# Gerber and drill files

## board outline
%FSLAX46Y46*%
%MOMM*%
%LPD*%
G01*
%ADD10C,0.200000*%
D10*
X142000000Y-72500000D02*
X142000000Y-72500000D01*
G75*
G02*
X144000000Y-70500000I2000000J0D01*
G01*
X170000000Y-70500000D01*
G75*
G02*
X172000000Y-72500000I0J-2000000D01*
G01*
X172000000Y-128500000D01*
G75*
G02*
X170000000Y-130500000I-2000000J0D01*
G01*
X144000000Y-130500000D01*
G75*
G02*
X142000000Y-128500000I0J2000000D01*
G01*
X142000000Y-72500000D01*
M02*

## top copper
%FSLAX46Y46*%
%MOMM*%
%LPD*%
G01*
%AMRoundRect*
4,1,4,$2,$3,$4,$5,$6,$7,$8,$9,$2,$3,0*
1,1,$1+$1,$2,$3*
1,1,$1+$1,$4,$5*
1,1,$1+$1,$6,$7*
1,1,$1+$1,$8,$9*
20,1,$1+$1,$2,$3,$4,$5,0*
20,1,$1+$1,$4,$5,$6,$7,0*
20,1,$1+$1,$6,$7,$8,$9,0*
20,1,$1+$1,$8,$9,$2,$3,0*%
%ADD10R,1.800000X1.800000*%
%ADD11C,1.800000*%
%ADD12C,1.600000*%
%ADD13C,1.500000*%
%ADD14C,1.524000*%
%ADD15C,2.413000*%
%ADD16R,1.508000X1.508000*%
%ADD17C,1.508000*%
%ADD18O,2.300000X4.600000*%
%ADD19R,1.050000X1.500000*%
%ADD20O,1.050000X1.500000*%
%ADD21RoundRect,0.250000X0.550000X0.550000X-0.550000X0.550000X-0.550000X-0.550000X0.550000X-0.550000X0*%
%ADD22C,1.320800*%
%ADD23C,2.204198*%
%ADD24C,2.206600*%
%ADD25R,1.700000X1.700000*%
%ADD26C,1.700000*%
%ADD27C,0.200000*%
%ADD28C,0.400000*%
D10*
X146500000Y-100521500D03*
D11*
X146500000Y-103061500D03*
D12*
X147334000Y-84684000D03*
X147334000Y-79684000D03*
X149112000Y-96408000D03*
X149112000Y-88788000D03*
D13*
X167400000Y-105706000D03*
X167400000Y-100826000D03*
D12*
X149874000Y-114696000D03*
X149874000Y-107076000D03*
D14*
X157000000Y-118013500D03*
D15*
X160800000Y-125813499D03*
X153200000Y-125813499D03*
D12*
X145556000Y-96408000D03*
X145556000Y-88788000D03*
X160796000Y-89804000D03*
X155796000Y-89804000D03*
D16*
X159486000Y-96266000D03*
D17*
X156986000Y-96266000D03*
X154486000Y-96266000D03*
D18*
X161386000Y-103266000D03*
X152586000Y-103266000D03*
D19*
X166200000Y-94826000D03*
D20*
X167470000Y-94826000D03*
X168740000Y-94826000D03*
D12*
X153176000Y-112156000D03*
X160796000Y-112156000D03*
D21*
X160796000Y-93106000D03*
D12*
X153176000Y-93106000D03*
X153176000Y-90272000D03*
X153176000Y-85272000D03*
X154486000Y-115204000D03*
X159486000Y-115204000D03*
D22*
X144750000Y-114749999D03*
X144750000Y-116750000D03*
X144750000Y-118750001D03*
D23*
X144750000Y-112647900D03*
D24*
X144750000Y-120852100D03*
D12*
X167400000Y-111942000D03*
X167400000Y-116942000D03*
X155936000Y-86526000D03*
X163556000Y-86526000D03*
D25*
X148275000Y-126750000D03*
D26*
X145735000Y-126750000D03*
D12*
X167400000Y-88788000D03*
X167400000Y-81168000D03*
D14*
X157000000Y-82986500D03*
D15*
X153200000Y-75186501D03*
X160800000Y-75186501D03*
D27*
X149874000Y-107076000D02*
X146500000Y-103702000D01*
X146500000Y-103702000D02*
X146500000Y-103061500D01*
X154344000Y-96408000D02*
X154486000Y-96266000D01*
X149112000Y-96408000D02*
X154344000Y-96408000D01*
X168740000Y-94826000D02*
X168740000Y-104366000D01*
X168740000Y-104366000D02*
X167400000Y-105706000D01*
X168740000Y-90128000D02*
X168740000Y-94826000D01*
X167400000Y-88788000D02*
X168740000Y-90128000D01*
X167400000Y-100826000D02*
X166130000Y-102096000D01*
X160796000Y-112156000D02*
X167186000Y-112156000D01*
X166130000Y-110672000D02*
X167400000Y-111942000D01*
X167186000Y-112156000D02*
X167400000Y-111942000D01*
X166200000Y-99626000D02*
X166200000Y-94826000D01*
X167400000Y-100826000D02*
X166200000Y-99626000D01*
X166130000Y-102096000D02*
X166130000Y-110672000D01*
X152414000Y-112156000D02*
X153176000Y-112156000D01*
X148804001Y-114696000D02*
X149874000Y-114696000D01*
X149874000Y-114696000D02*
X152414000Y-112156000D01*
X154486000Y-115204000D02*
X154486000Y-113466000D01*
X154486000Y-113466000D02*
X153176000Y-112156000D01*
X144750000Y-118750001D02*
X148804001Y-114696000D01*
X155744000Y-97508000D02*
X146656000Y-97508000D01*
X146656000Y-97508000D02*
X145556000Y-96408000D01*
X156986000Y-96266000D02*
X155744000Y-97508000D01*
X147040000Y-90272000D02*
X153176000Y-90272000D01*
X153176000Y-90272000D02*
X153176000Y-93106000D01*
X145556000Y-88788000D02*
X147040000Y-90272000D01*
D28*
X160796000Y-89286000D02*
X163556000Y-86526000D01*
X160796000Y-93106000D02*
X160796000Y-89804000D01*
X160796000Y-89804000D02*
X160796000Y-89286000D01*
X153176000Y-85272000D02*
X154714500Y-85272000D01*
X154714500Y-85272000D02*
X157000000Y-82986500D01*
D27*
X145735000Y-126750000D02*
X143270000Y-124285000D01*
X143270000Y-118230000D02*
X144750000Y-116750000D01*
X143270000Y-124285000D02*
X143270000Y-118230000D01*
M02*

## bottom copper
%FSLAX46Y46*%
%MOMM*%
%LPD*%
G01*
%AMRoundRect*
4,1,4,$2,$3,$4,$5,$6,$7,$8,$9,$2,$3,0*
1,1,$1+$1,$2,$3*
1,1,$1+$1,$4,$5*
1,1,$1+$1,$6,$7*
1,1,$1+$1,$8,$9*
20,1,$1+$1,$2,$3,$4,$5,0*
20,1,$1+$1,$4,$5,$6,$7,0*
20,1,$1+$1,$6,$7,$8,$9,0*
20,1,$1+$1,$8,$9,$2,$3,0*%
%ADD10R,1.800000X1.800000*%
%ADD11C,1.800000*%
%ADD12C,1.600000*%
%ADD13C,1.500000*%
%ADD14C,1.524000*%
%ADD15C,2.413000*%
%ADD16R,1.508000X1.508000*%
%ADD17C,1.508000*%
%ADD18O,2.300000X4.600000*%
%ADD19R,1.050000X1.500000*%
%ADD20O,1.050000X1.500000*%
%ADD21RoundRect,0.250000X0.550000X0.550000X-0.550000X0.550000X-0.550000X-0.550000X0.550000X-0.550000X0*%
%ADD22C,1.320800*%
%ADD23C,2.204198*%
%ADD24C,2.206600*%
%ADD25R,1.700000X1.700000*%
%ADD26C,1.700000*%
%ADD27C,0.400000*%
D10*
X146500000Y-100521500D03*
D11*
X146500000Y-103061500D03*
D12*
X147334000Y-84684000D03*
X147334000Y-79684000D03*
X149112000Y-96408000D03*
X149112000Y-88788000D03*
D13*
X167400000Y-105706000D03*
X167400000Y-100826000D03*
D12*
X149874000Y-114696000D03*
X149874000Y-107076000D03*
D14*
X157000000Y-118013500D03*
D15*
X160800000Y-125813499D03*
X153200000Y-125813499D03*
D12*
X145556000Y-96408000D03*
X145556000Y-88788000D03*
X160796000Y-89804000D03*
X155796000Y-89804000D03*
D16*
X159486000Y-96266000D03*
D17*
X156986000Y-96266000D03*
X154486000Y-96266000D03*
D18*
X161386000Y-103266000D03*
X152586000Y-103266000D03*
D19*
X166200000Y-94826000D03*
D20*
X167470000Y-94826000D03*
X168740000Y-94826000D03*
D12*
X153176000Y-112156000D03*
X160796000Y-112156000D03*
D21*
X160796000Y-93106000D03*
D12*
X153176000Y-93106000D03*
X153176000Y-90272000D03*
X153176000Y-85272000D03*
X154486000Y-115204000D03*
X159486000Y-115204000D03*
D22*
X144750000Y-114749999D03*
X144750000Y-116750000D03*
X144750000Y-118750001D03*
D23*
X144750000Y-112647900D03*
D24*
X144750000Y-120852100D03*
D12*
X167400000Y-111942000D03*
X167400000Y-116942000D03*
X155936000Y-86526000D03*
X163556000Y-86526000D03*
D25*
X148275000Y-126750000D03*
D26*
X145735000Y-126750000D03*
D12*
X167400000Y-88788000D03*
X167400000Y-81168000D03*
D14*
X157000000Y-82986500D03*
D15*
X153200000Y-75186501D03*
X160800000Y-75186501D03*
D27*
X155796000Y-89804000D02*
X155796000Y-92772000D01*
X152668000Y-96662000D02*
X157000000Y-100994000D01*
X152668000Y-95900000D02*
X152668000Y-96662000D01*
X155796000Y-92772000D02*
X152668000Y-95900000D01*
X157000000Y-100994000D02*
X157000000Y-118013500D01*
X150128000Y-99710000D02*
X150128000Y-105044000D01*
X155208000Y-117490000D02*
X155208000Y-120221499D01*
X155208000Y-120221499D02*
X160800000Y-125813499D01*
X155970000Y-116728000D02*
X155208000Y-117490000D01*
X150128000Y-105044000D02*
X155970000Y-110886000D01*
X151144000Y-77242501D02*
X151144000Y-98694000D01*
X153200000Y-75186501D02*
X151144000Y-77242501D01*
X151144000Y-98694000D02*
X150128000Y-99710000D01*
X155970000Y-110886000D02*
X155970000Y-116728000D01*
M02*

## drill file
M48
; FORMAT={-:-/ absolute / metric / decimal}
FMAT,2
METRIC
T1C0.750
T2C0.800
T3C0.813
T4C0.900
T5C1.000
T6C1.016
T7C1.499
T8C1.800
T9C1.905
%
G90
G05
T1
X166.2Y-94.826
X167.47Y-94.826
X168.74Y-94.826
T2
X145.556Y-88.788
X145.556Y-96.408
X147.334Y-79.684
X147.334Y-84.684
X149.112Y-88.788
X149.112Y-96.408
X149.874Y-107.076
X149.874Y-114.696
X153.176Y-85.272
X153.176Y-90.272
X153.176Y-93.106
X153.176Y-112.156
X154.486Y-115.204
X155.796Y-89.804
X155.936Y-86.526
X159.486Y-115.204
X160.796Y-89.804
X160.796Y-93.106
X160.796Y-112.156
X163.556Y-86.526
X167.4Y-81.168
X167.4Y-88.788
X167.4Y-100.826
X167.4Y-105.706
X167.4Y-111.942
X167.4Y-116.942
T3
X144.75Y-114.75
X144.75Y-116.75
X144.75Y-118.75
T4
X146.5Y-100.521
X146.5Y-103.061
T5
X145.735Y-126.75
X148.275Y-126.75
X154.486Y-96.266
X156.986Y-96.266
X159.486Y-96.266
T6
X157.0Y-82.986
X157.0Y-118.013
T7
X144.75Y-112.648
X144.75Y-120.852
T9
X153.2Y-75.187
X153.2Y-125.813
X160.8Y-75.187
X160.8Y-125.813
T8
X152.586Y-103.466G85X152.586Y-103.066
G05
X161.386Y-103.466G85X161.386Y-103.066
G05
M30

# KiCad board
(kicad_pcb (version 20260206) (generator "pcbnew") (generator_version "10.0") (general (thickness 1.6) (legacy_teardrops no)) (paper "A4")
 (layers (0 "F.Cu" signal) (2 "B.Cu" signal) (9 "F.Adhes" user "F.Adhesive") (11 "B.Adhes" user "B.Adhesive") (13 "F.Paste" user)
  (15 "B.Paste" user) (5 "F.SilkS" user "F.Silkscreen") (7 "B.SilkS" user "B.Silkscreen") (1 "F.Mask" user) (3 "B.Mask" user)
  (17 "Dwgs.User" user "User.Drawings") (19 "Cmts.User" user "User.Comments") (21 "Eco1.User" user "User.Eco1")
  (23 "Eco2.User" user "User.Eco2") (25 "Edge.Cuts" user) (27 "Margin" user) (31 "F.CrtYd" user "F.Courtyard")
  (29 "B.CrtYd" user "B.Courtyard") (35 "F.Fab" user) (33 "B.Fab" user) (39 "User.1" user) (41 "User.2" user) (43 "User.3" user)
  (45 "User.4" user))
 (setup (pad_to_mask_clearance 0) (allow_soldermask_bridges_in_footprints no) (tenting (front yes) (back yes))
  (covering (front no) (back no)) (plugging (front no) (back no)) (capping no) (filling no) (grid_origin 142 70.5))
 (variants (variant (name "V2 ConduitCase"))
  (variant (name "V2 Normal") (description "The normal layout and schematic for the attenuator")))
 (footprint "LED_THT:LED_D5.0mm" (layer "F.Cu") (at 146.5 100.5215 -90)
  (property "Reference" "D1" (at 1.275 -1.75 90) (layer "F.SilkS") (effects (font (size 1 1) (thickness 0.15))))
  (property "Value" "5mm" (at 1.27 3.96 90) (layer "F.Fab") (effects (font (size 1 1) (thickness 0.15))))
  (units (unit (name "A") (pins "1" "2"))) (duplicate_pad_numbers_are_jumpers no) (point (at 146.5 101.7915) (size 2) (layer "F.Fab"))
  (pad "1" thru_hole rect (at 0 0 270) (size 1.8 1.8) (drill 0.9) (layers "*.Cu" "*.Mask") (remove_unused_layers no) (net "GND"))
  (pad "2" thru_hole circle (at 2.54 0 270) (size 1.8 1.8) (drill 0.9) (layers "*.Cu" "*.Mask") (remove_unused_layers no) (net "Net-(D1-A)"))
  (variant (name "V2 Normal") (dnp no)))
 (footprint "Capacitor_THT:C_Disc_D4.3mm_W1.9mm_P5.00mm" (layer "F.Cu") (at 147.334 84.684 90)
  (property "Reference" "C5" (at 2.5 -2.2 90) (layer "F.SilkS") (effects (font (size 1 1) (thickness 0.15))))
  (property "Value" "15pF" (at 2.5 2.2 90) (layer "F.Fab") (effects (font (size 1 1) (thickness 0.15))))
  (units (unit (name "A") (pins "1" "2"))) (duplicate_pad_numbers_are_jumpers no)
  (pad "1" thru_hole circle (at 0 0 90) (size 1.6 1.6) (drill 0.8) (layers "*.Cu" "*.Mask") (remove_unused_layers no) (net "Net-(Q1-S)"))
  (pad "2" thru_hole circle (at 5 0 90) (size 1.6 1.6) (drill 0.8) (layers "*.Cu" "*.Mask") (remove_unused_layers no) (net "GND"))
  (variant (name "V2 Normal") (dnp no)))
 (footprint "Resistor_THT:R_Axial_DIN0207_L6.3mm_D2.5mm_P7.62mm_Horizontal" (layer "F.Cu") (at 149.112 96.408 90)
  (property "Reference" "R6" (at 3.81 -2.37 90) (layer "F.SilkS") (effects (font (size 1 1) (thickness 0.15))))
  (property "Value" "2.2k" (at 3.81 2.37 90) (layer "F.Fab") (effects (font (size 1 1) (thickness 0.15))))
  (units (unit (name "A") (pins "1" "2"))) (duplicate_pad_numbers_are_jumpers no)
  (pad "1" thru_hole circle (at 0 0 90) (size 1.6 1.6) (drill 0.8) (layers "*.Cu" "*.Mask") (remove_unused_layers no) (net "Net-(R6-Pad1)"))
  (pad "2" thru_hole circle (at 7.62 0 90) (size 1.6 1.6) (drill 0.8) (layers "*.Cu" "*.Mask") (remove_unused_layers no) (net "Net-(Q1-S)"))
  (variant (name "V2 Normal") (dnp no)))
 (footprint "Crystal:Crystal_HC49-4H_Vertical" (layer "F.Cu") (at 167.4 105.706 90)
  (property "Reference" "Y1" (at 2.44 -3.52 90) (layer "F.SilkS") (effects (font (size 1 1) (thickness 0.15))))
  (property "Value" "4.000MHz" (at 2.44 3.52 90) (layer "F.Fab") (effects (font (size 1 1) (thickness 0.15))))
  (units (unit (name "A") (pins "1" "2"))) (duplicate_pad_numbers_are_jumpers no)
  (pad "1" thru_hole circle (at 0 0 90) (size 1.5 1.5) (drill 0.8) (layers "*.Cu" "*.Mask") (remove_unused_layers no) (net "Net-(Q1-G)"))
  (pad "2" thru_hole circle (at 4.88 0 90) (size 1.5 1.5) (drill 0.8) (layers "*.Cu" "*.Mask") (remove_unused_layers no) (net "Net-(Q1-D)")))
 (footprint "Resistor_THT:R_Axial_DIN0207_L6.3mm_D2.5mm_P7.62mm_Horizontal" (layer "F.Cu") (at 149.874 114.696 90)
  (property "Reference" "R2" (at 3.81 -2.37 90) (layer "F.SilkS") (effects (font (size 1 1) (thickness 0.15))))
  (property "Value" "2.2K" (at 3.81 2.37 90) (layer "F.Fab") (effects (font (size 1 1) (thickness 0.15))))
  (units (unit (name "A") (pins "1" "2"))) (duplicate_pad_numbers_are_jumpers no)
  (pad "1" thru_hole circle (at 0 0 90) (size 1.6 1.6) (drill 0.8) (layers "*.Cu" "*.Mask") (remove_unused_layers no) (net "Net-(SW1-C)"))
  (pad "2" thru_hole circle (at 7.62 0 90) (size 1.6 1.6) (drill 0.8) (layers "*.Cu" "*.Mask") (remove_unused_layers no) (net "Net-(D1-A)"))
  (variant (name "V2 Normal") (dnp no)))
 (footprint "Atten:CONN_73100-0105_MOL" (layer "F.Cu") (at 157 118.0135 180)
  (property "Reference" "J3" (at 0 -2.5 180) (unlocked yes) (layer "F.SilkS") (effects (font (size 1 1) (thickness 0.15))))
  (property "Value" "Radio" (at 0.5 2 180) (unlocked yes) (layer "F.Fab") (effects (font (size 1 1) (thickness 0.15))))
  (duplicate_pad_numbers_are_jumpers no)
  (pad "1" thru_hole circle (at 0 0 180) (size 1.524 1.524) (drill 1.016) (layers "*.Cu" "*.Mask") (remove_unused_layers no)
   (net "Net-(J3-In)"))
  (pad "2" thru_hole circle (at -3.8 -7.799999 180) (size 2.413 2.413) (drill 1.905) (layers "*.Cu" "*.Mask") (remove_unused_layers no)
   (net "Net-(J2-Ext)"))
  (pad "3" thru_hole circle (at 3.8 -7.799999 180) (size 2.413 2.413) (drill 1.905) (layers "*.Cu" "*.Mask") (remove_unused_layers no)))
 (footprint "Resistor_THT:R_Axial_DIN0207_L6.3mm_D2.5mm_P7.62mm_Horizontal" (layer "F.Cu") (at 145.556 96.408 90)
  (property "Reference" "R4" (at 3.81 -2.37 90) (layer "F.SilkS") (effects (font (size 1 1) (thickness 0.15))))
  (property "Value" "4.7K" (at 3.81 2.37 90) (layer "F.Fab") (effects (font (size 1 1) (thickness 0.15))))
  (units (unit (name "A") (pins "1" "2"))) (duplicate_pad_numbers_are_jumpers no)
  (pad "1" thru_hole circle (at 0 0 90) (size 1.6 1.6) (drill 0.8) (layers "*.Cu" "*.Mask") (remove_unused_layers no) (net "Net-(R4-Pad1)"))
  (pad "2" thru_hole circle (at 7.62 0 90) (size 1.6 1.6) (drill 0.8) (layers "*.Cu" "*.Mask") (remove_unused_layers no) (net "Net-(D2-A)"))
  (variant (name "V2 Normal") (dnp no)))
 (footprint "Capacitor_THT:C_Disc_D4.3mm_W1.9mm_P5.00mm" (layer "F.Cu") (at 160.796 89.804 180)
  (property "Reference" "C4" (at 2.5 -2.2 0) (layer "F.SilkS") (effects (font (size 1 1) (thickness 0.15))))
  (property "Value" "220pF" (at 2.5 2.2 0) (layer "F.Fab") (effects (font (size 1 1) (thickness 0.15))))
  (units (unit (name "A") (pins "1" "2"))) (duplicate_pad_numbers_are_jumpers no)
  (pad "1" thru_hole circle (at 0 0 180) (size 1.6 1.6) (drill 0.8) (layers "*.Cu" "*.Mask") (remove_unused_layers no) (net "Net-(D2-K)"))
  (pad "2" thru_hole circle (at 5 0 180) (size 1.6 1.6) (drill 0.8) (layers "*.Cu" "*.Mask") (remove_unused_layers no) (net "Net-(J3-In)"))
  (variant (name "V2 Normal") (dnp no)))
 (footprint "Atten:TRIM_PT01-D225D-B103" (layer "F.Cu") (at 156.986 103.266 180)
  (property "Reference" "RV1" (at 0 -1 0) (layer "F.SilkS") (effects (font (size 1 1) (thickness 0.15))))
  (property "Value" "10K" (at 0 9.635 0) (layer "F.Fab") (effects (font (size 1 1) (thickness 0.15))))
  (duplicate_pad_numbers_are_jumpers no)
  (pad "1" thru_hole rect (at -2.5 7 180) (size 1.508 1.508) (drill 1) (layers "*.Cu" "*.Mask") (remove_unused_layers no) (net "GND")
   (solder_mask_margin 0.102))
  (pad "2" thru_hole circle (at 0 7 180) (size 1.508 1.508) (drill 1) (layers "*.Cu" "*.Mask") (remove_unused_layers no)
   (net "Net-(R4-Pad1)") (solder_mask_margin 0.102))
  (pad "3" thru_hole circle (at 2.5 7 180) (size 1.508 1.508) (drill 1) (layers "*.Cu" "*.Mask") (remove_unused_layers no)
   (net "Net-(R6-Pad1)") (solder_mask_margin 0.102))
  (pad "MP" thru_hole oval (at -4.4 0 180) (size 2.3 4.6) (drill oval 1.8 2.2) (layers "*.Cu" "*.Mask") (remove_unused_layers no)
   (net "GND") (solder_mask_margin 0.102))
  (pad "MP" thru_hole oval (at 4.4 0 180) (size 2.3 4.6) (drill oval 1.8 2.2) (layers "*.Cu" "*.Mask") (remove_unused_layers no) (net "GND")
   (solder_mask_margin 0.102)))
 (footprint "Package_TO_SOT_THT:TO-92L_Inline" (layer "F.Cu") (at 166.2 94.826)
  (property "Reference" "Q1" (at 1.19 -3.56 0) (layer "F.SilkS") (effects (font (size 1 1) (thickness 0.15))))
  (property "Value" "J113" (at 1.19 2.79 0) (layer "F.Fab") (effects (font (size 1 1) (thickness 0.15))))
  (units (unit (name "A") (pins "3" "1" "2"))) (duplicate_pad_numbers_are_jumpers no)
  (pad "1" thru_hole rect (at 0 0) (size 1.05 1.5) (drill 0.75) (layers "*.Cu" "*.Mask") (remove_unused_layers no) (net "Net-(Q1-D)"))
  (pad "2" thru_hole oval (at 1.27 0) (size 1.05 1.5) (drill 0.75) (layers "*.Cu" "*.Mask") (remove_unused_layers no) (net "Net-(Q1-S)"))
  (pad "3" thru_hole oval (at 2.54 0) (size 1.05 1.5) (drill 0.75) (layers "*.Cu" "*.Mask") (remove_unused_layers no) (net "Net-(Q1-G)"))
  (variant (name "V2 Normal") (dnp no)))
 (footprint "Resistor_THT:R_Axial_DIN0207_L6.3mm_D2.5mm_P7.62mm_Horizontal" (layer "F.Cu") (at 153.176 112.156)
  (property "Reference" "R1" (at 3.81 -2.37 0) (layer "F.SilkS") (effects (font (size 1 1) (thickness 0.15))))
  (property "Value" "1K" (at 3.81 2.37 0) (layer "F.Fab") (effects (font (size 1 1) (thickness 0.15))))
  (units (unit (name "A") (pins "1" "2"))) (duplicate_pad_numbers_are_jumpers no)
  (pad "1" thru_hole circle (at 0 0) (size 1.6 1.6) (drill 0.8) (layers "*.Cu" "*.Mask") (remove_unused_layers no) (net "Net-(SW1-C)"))
  (pad "2" thru_hole circle (at 7.62 0) (size 1.6 1.6) (drill 0.8) (layers "*.Cu" "*.Mask") (remove_unused_layers no) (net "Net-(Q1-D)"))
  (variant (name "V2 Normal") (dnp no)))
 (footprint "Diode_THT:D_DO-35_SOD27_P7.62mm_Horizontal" (layer "F.Cu") (at 160.796 93.106 180)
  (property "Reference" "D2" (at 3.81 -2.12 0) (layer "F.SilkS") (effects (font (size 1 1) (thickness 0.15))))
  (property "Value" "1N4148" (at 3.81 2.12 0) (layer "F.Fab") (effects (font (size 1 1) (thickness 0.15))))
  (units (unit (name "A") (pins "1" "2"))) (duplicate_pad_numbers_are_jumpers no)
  (pad "1" thru_hole roundrect (at 0 0 180) (size 1.6 1.6) (drill 0.8) (layers "*.Cu" "*.Mask") (remove_unused_layers no)
   (roundrect_rratio 0.15625) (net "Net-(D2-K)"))
  (pad "2" thru_hole circle (at 7.62 0 180) (size 1.6 1.6) (drill 0.8) (layers "*.Cu" "*.Mask") (remove_unused_layers no) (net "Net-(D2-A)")))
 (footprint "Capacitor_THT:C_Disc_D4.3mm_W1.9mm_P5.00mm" (layer "F.Cu") (at 153.176 90.272 90)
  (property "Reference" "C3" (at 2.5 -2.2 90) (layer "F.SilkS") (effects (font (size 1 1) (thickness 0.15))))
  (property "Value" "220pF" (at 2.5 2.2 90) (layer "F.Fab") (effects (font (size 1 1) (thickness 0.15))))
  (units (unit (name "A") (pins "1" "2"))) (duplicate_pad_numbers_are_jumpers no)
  (pad "1" thru_hole circle (at 0 0 90) (size 1.6 1.6) (drill 0.8) (layers "*.Cu" "*.Mask") (remove_unused_layers no) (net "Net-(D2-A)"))
  (pad "2" thru_hole circle (at 5 0 90) (size 1.6 1.6) (drill 0.8) (layers "*.Cu" "*.Mask") (remove_unused_layers no) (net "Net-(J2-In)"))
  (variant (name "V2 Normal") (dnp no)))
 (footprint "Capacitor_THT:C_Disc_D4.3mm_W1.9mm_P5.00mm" (layer "F.Cu") (at 154.486 115.204)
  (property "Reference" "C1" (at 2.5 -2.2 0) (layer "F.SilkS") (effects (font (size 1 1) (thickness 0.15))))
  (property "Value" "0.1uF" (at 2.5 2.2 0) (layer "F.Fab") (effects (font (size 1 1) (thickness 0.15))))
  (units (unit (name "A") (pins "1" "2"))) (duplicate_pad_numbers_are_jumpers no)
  (pad "1" thru_hole circle (at 0 0) (size 1.6 1.6) (drill 0.8) (layers "*.Cu" "*.Mask") (remove_unused_layers no) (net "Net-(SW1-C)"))
  (pad "2" thru_hole circle (at 5 0) (size 1.6 1.6) (drill 0.8) (layers "*.Cu" "*.Mask") (remove_unused_layers no) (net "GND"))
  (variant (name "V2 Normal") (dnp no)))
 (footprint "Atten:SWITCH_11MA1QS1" (layer "F.Cu") (at 144.75 114.749999 -90)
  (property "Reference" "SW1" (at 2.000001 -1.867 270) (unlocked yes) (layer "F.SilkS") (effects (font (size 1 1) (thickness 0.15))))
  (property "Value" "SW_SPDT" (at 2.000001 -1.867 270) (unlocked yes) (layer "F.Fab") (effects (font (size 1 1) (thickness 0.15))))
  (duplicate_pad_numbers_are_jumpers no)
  (pad "1" thru_hole circle (at 0 0 270) (size 1.3208 1.3208) (drill 0.8128) (layers "*.Cu" "*.Mask") (remove_unused_layers no)
   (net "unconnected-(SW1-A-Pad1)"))
  (pad "2" thru_hole circle (at 2.000001 0 270) (size 1.3208 1.3208) (drill 0.8128) (layers "*.Cu" "*.Mask") (remove_unused_layers no)
   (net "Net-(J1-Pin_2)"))
  (pad "3" thru_hole circle (at 4.000002 0 270) (size 1.3208 1.3208) (drill 0.8128) (layers "*.Cu" "*.Mask") (remove_unused_layers no)
   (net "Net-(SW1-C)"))
  (pad "4" thru_hole circle (at -2.102099 0 270) (size 2.204198 2.204198) (drill 1.4986) (layers "*.Cu" "*.Mask") (remove_unused_layers no))
  (pad "5" thru_hole circle (at 6.102101 0 270) (size 2.2066 2.2066) (drill 1.4986) (layers "*.Cu" "*.Mask") (remove_unused_layers no)))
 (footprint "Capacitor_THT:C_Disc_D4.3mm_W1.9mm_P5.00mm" (layer "F.Cu") (at 167.4 111.942 -90)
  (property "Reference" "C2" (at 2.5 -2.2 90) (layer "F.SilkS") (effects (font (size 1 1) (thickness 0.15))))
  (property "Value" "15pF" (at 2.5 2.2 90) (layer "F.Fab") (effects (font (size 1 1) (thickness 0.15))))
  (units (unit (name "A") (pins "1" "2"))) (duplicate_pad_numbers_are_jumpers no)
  (pad "1" thru_hole circle (at 0 0 270) (size 1.6 1.6) (drill 0.8) (layers "*.Cu" "*.Mask") (remove_unused_layers no) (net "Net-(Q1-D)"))
  (pad "2" thru_hole circle (at 5 0 270) (size 1.6 1.6) (drill 0.8) (layers "*.Cu" "*.Mask") (remove_unused_layers no) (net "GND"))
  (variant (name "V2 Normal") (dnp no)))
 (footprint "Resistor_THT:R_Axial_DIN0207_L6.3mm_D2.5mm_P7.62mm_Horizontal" (layer "F.Cu") (at 155.936 86.526)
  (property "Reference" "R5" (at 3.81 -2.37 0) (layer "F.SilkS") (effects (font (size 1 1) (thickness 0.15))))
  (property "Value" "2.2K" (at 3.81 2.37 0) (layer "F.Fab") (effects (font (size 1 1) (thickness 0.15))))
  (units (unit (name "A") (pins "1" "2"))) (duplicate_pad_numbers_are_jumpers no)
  (pad "1" thru_hole circle (at 0 0) (size 1.6 1.6) (drill 0.8) (layers "*.Cu" "*.Mask") (remove_unused_layers no) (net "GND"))
  (pad "2" thru_hole circle (at 7.62 0) (size 1.6 1.6) (drill 0.8) (layers "*.Cu" "*.Mask") (remove_unused_layers no) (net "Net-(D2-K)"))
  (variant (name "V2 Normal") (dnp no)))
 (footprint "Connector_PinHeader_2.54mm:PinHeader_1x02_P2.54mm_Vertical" (layer "F.Cu") (at 148.275 126.75 -90)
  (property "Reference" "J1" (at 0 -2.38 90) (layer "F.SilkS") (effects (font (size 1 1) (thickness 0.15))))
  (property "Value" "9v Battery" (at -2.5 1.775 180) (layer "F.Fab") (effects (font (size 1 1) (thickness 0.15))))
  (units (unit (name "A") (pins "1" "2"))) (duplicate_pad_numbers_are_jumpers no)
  (pad "1" thru_hole rect (at 0 0 270) (size 1.7 1.7) (drill 1) (layers "*.Cu" "*.Mask") (remove_unused_layers no) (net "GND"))
  (pad "2" thru_hole circle (at 0 2.54 270) (size 1.7 1.7) (drill 1) (layers "*.Cu" "*.Mask") (remove_unused_layers no)
   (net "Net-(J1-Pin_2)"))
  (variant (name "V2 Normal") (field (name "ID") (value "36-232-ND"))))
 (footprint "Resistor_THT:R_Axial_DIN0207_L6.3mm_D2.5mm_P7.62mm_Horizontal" (layer "F.Cu") (at 167.4 88.788 90)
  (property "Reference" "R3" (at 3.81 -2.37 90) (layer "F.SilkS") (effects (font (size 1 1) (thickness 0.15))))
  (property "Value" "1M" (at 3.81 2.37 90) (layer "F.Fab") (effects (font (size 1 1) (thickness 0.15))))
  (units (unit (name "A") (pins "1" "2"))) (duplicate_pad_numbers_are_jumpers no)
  (pad "1" thru_hole circle (at 0 0 90) (size 1.6 1.6) (drill 0.8) (layers "*.Cu" "*.Mask") (remove_unused_layers no) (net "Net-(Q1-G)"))
  (pad "2" thru_hole circle (at 7.62 0 90) (size 1.6 1.6) (drill 0.8) (layers "*.Cu" "*.Mask") (remove_unused_layers no) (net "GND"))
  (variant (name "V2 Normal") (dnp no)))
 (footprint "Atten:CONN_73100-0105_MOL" (layer "F.Cu") (at 157 82.9865)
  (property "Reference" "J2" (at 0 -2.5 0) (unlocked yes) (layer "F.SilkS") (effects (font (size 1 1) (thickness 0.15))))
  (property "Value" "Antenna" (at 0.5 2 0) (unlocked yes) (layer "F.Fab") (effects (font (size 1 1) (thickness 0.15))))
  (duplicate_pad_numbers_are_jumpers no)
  (pad "1" thru_hole circle (at 0 0) (size 1.524 1.524) (drill 1.016) (layers "*.Cu" "*.Mask") (remove_unused_layers no) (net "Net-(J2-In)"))
  (pad "2" thru_hole circle (at -3.8 -7.799999) (size 2.413 2.413) (drill 1.905) (layers "*.Cu" "*.Mask") (remove_unused_layers no)
   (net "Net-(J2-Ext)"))
  (pad "3" thru_hole circle (at 3.8 -7.799999) (size 2.413 2.413) (drill 1.905) (layers "*.Cu" "*.Mask") (remove_unused_layers no)))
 (gr_rect (start 142 70.5) (end 172 130.5) (radius 2) (stroke (width 0.2) (type solid)) (fill no) (layer "Edge.Cuts"))
 (segment (start 149.874 107.076) (end 146.5 103.702) (width 0.2) (layer "F.Cu") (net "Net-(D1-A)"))
 (segment (start 146.5 103.702) (end 146.5 103.0615) (width 0.2) (layer "F.Cu") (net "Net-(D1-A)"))
 (segment (start 154.344 96.408) (end 154.486 96.266) (width 0.2) (layer "F.Cu") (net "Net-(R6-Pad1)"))
 (segment (start 149.112 96.408) (end 154.344 96.408) (width 0.2) (layer "F.Cu") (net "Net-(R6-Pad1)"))
 (segment (start 168.74 94.826) (end 168.74 104.366) (width 0.2) (layer "F.Cu") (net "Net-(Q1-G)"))
 (segment (start 168.74 104.366) (end 167.4 105.706) (width 0.2) (layer "F.Cu") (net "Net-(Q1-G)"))
 (segment (start 168.74 90.128) (end 168.74 94.826) (width 0.2) (layer "F.Cu") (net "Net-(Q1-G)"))
 (segment (start 167.4 88.788) (end 168.74 90.128) (width 0.2) (layer "F.Cu") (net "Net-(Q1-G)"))
 (segment (start 167.4 100.826) (end 166.13 102.096) (width 0.2) (layer "F.Cu") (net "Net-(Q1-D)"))
 (segment (start 160.796 112.156) (end 167.186 112.156) (width 0.2) (layer "F.Cu") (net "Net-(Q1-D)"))
 (segment (start 166.13 110.672) (end 167.4 111.942) (width 0.2) (layer "F.Cu") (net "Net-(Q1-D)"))
 (segment (start 167.186 112.156) (end 167.4 111.942) (width 0.2) (layer "F.Cu") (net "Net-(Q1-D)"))
 (segment (start 166.2 99.626) (end 166.2 94.826) (width 0.2) (layer "F.Cu") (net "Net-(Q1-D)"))
 (segment (start 167.4 100.826) (end 166.2 99.626) (width 0.2) (layer "F.Cu") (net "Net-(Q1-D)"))
 (segment (start 166.13 102.096) (end 166.13 110.672) (width 0.2) (layer "F.Cu") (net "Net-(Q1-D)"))
 (segment (start 152.414 112.156) (end 153.176 112.156) (width 0.2) (layer "F.Cu") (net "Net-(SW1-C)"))
 (segment (start 148.804001 114.696) (end 149.874 114.696) (width 0.2) (layer "F.Cu") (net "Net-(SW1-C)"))
 (segment (start 149.874 114.696) (end 152.414 112.156) (width 0.2) (layer "F.Cu") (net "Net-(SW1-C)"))
 (segment (start 154.486 115.204) (end 154.486 113.466) (width 0.2) (layer "F.Cu") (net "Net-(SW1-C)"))
 (segment (start 154.486 113.466) (end 153.176 112.156) (width 0.2) (layer "F.Cu") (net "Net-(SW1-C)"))
 (segment (start 144.75 118.750001) (end 148.804001 114.696) (width 0.2) (layer "F.Cu") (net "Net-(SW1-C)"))
 (segment (start 155.796 89.804) (end 155.796 92.772) (width 0.4) (layer "B.Cu") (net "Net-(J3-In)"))
 (segment (start 152.668 96.662) (end 157 100.994) (width 0.4) (layer "B.Cu") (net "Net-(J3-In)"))
 (segment (start 152.668 95.9) (end 152.668 96.662) (width 0.4) (layer "B.Cu") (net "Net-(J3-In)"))
 (segment (start 155.796 92.772) (end 152.668 95.9) (width 0.4) (layer "B.Cu") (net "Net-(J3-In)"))
 (segment (start 157 100.994) (end 157 118.0135) (width 0.4) (layer "B.Cu") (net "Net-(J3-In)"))
 (segment (start 150.128 99.71) (end 150.128 105.044) (width 0.4) (layer "B.Cu") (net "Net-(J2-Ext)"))
 (segment (start 155.208 117.49) (end 155.208 120.221499) (width 0.4) (layer "B.Cu") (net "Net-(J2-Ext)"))
 (segment (start 155.208 120.221499) (end 160.8 125.813499) (width 0.4) (layer "B.Cu") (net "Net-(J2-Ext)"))
 (segment (start 155.97 116.728) (end 155.208 117.49) (width 0.4) (layer "B.Cu") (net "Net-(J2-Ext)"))
 (segment (start 150.128 105.044) (end 155.97 110.886) (width 0.4) (layer "B.Cu") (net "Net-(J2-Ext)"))
 (segment (start 151.144 77.242501) (end 151.144 98.694) (width 0.4) (layer "B.Cu") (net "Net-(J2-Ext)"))
 (segment (start 153.2 75.186501) (end 151.144 77.242501) (width 0.4) (layer "B.Cu") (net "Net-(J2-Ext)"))
 (segment (start 151.144 98.694) (end 150.128 99.71) (width 0.4) (layer "B.Cu") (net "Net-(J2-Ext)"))
 (segment (start 155.97 110.886) (end 155.97 116.728) (width 0.4) (layer "B.Cu") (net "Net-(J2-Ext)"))
 (segment (start 155.744 97.508) (end 146.656 97.508) (width 0.2) (layer "F.Cu") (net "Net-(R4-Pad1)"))
 (segment (start 146.656 97.508) (end 145.556 96.408) (width 0.2) (layer "F.Cu") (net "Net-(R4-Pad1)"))
 (segment (start 156.986 96.266) (end 155.744 97.508) (width 0.2) (layer "F.Cu") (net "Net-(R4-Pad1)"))
 (segment (start 147.04 90.272) (end 153.176 90.272) (width 0.2) (layer "F.Cu") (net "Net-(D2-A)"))
 (segment (start 153.176 90.272) (end 153.176 93.106) (width 0.2) (layer "F.Cu") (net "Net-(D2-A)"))
 (segment (start 145.556 88.788) (end 147.04 90.272) (width 0.2) (layer "F.Cu") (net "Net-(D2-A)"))
 (segment (start 160.796 89.286) (end 163.556 86.526) (width 0.4) (layer "F.Cu") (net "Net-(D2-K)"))
 (segment (start 160.796 93.106) (end 160.796 89.804) (width 0.4) (layer "F.Cu") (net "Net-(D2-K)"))
 (segment (start 160.796 89.804) (end 160.796 89.286) (width 0.4) (layer "F.Cu") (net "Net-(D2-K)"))
 (segment (start 153.176 85.272) (end 154.7145 85.272) (width 0.4) (layer "F.Cu") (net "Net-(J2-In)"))
 (segment (start 154.7145 85.272) (end 157 82.9865) (width 0.4) (layer "F.Cu") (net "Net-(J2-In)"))
 (segment (start 145.735 126.75) (end 143.27 124.285) (width 0.2) (layer "F.Cu") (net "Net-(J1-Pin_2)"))
 (segment (start 143.27 118.23) (end 144.75 116.75) (width 0.2) (layer "F.Cu") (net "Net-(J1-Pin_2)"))
 (segment (start 143.27 124.285) (end 143.27 118.23) (width 0.2) (layer "F.Cu") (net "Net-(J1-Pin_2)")))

